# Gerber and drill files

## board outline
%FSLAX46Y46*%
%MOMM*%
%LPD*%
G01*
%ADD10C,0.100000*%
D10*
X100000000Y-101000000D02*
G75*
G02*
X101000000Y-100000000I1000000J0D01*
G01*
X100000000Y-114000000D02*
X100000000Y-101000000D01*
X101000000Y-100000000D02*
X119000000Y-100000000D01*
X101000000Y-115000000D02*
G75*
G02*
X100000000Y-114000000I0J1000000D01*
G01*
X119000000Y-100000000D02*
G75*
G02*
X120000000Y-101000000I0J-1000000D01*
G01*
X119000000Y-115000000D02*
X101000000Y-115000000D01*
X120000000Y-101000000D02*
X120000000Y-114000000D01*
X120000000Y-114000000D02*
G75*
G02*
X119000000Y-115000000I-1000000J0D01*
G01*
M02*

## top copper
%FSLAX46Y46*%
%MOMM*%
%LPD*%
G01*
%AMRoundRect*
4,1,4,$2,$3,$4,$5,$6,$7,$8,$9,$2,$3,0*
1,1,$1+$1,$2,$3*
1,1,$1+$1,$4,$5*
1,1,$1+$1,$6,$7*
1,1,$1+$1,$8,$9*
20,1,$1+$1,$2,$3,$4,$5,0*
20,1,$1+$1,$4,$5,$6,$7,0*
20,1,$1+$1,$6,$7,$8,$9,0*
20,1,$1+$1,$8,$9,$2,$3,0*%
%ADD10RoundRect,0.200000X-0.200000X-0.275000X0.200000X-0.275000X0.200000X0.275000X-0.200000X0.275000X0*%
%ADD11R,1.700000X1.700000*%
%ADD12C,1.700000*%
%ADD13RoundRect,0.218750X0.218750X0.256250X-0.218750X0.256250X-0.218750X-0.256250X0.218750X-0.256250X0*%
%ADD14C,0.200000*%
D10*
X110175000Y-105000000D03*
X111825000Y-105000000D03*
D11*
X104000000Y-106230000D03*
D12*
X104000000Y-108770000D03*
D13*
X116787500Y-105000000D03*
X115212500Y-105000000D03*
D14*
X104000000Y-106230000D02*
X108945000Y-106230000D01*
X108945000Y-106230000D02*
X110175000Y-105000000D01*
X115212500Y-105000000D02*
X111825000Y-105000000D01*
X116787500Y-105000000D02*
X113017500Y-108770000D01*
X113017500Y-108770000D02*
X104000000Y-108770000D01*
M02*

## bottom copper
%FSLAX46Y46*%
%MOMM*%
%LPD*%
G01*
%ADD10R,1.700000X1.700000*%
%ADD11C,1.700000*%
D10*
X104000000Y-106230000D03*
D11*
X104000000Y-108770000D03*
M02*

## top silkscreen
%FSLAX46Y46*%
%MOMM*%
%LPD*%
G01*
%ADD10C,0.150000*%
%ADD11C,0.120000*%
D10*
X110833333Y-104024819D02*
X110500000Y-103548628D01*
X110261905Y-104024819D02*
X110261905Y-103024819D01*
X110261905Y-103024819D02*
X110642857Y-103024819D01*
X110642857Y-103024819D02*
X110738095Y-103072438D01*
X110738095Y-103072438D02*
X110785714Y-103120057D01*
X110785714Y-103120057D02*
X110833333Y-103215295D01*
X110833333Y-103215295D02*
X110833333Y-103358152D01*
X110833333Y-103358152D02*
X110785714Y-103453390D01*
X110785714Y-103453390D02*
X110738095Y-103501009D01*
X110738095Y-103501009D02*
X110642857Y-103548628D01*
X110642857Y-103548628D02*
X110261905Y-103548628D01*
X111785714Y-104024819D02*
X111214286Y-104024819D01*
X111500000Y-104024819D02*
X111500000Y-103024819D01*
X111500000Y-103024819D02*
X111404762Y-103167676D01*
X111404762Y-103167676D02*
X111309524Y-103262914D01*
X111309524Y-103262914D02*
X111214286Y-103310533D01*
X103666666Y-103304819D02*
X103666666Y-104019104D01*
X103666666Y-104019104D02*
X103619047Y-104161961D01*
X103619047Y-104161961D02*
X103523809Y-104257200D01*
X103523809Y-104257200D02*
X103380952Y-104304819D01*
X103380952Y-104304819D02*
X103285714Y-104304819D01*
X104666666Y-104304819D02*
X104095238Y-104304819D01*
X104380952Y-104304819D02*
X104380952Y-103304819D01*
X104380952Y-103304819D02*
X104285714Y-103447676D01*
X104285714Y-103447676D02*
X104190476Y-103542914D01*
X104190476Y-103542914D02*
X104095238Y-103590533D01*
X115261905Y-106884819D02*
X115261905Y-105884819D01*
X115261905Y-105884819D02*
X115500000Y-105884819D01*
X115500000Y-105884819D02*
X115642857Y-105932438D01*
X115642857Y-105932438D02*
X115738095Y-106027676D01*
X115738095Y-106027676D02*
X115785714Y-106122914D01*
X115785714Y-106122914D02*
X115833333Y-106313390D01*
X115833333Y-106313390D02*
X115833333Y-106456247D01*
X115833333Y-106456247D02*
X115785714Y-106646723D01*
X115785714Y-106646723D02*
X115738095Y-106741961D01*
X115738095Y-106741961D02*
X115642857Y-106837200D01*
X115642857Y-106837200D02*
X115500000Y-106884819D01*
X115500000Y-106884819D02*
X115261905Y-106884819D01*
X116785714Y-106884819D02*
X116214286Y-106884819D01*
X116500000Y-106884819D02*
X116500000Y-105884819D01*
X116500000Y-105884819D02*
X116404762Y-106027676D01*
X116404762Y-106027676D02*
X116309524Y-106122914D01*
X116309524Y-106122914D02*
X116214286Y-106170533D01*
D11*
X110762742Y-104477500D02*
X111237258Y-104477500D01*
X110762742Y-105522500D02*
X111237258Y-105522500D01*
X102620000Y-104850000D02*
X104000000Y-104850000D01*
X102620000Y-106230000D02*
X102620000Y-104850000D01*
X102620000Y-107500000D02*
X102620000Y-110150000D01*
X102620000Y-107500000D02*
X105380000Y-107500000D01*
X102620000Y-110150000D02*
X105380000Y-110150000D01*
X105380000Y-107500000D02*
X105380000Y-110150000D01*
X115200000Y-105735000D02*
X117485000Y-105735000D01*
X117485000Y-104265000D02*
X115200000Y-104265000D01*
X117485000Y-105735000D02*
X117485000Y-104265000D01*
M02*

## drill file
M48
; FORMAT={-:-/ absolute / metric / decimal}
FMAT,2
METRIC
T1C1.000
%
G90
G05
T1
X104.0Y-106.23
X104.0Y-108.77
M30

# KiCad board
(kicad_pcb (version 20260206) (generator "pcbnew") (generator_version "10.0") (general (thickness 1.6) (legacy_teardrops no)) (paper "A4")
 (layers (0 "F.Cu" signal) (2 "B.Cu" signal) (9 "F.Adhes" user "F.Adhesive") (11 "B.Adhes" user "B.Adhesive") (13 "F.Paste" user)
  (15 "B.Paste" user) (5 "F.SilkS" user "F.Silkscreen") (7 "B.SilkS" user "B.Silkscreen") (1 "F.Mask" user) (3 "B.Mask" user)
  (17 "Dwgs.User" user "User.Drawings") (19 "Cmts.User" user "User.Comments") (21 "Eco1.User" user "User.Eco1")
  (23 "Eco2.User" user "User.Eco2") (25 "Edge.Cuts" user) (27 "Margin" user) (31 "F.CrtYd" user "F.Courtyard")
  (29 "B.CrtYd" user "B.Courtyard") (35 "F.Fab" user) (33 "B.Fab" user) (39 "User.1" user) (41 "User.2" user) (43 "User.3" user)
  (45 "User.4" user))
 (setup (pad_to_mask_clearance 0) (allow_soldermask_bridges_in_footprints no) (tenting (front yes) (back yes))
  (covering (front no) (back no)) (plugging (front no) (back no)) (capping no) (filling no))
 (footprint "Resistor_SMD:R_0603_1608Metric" (layer "F.Cu") (at 111 105)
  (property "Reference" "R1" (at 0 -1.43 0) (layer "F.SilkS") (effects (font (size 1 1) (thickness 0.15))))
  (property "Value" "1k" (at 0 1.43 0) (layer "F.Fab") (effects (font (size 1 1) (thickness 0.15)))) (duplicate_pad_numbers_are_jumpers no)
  (fp_line (start -0.237258 -0.5225) (end 0.237258 -0.5225) (stroke (width 0.12) (type solid)) (layer "F.SilkS"))
  (fp_line (start -0.237258 0.5225) (end 0.237258 0.5225) (stroke (width 0.12) (type solid)) (layer "F.SilkS"))
  (pad "1" smd roundrect (at -0.825 0) (size 0.8 0.95) (layers "F.Cu" "F.Mask" "F.Paste") (roundrect_rratio 0.25) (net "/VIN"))
  (pad "2" smd roundrect (at 0.825 0) (size 0.8 0.95) (layers "F.Cu" "F.Mask" "F.Paste") (roundrect_rratio 0.25) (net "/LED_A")))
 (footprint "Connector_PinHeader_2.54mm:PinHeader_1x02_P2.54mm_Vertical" (layer "F.Cu") (at 104 106.23)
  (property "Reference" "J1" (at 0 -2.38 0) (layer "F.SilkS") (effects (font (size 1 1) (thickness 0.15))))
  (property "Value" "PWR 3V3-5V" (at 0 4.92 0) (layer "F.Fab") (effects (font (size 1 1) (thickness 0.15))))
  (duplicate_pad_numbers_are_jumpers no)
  (fp_line (start -1.38 -1.38) (end 0 -1.38) (stroke (width 0.12) (type solid)) (layer "F.SilkS"))
  (fp_line (start -1.38 0) (end -1.38 -1.38) (stroke (width 0.12) (type solid)) (layer "F.SilkS"))
  (fp_line (start -1.38 1.27) (end -1.38 3.92) (stroke (width 0.12) (type solid)) (layer "F.SilkS"))
  (fp_line (start -1.38 1.27) (end 1.38 1.27) (stroke (width 0.12) (type solid)) (layer "F.SilkS"))
  (fp_line (start -1.38 3.92) (end 1.38 3.92) (stroke (width 0.12) (type solid)) (layer "F.SilkS"))
  (fp_line (start 1.38 1.27) (end 1.38 3.92) (stroke (width 0.12) (type solid)) (layer "F.SilkS"))
  (pad "1" thru_hole rect (at 0 0) (size 1.7 1.7) (drill 1) (layers "*.Cu" "*.Mask") (remove_unused_layers no) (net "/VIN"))
  (pad "2" thru_hole circle (at 0 2.54) (size 1.7 1.7) (drill 1) (layers "*.Cu" "*.Mask") (remove_unused_layers no) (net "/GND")))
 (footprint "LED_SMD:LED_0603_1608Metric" (layer "F.Cu") (at 116 105 180)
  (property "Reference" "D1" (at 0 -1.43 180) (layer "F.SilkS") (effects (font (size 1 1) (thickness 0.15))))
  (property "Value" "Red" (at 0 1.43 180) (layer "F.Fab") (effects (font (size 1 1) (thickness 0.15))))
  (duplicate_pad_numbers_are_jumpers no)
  (fp_line (start 0.8 -0.735) (end -1.485 -0.735) (stroke (width 0.12) (type solid)) (layer "F.SilkS"))
  (fp_line (start -1.485 0.735) (end 0.8 0.735) (stroke (width 0.12) (type solid)) (layer "F.SilkS"))
  (fp_line (start -1.485 -0.735) (end -1.485 0.735) (stroke (width 0.12) (type solid)) (layer "F.SilkS"))
  (pad "1" smd roundrect (at -0.7875 0 180) (size 0.875 0.95) (layers "F.Cu" "F.Mask" "F.Paste") (roundrect_rratio 0.25) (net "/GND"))
  (pad "2" smd roundrect (at 0.7875 0 180) (size 0.875 0.95) (layers "F.Cu" "F.Mask" "F.Paste") (roundrect_rratio 0.25) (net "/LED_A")))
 (gr_arc (start 100 101) (mid 100.292893 100.292893) (end 101 100) (stroke (width 0.1) (type default)) (layer "Edge.Cuts"))
 (gr_line (start 100 114) (end 100 101) (stroke (width 0.1) (type default)) (layer "Edge.Cuts"))
 (gr_line (start 101 100) (end 119 100) (stroke (width 0.1) (type default)) (layer "Edge.Cuts"))
 (gr_arc (start 101 115) (mid 100.292893 114.707107) (end 100 114) (stroke (width 0.1) (type default)) (layer "Edge.Cuts"))
 (gr_arc (start 119 100) (mid 119.707107 100.292893) (end 120 101) (stroke (width 0.1) (type default)) (layer "Edge.Cuts"))
 (gr_line (start 119 115) (end 101 115) (stroke (width 0.1) (type default)) (layer "Edge.Cuts"))
 (gr_line (start 120 101) (end 120 114) (stroke (width 0.1) (type default)) (layer "Edge.Cuts"))
 (gr_arc (start 120 114) (mid 119.707107 114.707107) (end 119 115) (stroke (width 0.1) (type default)) (layer "Edge.Cuts"))
 (segment (start 104 106.23) (end 108.945 106.23) (width 0.2) (layer "F.Cu") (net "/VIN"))
 (segment (start 108.945 106.23) (end 110.175 105) (width 0.2) (layer "F.Cu") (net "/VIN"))
 (segment (start 115.2125 105) (end 111.825 105) (width 0.2) (layer "F.Cu") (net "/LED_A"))
 (segment (start 116.7875 105) (end 113.0175 108.77) (width 0.2) (layer "F.Cu") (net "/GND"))
 (segment (start 113.0175 108.77) (end 104 108.77) (width 0.2) (layer "F.Cu") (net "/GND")))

